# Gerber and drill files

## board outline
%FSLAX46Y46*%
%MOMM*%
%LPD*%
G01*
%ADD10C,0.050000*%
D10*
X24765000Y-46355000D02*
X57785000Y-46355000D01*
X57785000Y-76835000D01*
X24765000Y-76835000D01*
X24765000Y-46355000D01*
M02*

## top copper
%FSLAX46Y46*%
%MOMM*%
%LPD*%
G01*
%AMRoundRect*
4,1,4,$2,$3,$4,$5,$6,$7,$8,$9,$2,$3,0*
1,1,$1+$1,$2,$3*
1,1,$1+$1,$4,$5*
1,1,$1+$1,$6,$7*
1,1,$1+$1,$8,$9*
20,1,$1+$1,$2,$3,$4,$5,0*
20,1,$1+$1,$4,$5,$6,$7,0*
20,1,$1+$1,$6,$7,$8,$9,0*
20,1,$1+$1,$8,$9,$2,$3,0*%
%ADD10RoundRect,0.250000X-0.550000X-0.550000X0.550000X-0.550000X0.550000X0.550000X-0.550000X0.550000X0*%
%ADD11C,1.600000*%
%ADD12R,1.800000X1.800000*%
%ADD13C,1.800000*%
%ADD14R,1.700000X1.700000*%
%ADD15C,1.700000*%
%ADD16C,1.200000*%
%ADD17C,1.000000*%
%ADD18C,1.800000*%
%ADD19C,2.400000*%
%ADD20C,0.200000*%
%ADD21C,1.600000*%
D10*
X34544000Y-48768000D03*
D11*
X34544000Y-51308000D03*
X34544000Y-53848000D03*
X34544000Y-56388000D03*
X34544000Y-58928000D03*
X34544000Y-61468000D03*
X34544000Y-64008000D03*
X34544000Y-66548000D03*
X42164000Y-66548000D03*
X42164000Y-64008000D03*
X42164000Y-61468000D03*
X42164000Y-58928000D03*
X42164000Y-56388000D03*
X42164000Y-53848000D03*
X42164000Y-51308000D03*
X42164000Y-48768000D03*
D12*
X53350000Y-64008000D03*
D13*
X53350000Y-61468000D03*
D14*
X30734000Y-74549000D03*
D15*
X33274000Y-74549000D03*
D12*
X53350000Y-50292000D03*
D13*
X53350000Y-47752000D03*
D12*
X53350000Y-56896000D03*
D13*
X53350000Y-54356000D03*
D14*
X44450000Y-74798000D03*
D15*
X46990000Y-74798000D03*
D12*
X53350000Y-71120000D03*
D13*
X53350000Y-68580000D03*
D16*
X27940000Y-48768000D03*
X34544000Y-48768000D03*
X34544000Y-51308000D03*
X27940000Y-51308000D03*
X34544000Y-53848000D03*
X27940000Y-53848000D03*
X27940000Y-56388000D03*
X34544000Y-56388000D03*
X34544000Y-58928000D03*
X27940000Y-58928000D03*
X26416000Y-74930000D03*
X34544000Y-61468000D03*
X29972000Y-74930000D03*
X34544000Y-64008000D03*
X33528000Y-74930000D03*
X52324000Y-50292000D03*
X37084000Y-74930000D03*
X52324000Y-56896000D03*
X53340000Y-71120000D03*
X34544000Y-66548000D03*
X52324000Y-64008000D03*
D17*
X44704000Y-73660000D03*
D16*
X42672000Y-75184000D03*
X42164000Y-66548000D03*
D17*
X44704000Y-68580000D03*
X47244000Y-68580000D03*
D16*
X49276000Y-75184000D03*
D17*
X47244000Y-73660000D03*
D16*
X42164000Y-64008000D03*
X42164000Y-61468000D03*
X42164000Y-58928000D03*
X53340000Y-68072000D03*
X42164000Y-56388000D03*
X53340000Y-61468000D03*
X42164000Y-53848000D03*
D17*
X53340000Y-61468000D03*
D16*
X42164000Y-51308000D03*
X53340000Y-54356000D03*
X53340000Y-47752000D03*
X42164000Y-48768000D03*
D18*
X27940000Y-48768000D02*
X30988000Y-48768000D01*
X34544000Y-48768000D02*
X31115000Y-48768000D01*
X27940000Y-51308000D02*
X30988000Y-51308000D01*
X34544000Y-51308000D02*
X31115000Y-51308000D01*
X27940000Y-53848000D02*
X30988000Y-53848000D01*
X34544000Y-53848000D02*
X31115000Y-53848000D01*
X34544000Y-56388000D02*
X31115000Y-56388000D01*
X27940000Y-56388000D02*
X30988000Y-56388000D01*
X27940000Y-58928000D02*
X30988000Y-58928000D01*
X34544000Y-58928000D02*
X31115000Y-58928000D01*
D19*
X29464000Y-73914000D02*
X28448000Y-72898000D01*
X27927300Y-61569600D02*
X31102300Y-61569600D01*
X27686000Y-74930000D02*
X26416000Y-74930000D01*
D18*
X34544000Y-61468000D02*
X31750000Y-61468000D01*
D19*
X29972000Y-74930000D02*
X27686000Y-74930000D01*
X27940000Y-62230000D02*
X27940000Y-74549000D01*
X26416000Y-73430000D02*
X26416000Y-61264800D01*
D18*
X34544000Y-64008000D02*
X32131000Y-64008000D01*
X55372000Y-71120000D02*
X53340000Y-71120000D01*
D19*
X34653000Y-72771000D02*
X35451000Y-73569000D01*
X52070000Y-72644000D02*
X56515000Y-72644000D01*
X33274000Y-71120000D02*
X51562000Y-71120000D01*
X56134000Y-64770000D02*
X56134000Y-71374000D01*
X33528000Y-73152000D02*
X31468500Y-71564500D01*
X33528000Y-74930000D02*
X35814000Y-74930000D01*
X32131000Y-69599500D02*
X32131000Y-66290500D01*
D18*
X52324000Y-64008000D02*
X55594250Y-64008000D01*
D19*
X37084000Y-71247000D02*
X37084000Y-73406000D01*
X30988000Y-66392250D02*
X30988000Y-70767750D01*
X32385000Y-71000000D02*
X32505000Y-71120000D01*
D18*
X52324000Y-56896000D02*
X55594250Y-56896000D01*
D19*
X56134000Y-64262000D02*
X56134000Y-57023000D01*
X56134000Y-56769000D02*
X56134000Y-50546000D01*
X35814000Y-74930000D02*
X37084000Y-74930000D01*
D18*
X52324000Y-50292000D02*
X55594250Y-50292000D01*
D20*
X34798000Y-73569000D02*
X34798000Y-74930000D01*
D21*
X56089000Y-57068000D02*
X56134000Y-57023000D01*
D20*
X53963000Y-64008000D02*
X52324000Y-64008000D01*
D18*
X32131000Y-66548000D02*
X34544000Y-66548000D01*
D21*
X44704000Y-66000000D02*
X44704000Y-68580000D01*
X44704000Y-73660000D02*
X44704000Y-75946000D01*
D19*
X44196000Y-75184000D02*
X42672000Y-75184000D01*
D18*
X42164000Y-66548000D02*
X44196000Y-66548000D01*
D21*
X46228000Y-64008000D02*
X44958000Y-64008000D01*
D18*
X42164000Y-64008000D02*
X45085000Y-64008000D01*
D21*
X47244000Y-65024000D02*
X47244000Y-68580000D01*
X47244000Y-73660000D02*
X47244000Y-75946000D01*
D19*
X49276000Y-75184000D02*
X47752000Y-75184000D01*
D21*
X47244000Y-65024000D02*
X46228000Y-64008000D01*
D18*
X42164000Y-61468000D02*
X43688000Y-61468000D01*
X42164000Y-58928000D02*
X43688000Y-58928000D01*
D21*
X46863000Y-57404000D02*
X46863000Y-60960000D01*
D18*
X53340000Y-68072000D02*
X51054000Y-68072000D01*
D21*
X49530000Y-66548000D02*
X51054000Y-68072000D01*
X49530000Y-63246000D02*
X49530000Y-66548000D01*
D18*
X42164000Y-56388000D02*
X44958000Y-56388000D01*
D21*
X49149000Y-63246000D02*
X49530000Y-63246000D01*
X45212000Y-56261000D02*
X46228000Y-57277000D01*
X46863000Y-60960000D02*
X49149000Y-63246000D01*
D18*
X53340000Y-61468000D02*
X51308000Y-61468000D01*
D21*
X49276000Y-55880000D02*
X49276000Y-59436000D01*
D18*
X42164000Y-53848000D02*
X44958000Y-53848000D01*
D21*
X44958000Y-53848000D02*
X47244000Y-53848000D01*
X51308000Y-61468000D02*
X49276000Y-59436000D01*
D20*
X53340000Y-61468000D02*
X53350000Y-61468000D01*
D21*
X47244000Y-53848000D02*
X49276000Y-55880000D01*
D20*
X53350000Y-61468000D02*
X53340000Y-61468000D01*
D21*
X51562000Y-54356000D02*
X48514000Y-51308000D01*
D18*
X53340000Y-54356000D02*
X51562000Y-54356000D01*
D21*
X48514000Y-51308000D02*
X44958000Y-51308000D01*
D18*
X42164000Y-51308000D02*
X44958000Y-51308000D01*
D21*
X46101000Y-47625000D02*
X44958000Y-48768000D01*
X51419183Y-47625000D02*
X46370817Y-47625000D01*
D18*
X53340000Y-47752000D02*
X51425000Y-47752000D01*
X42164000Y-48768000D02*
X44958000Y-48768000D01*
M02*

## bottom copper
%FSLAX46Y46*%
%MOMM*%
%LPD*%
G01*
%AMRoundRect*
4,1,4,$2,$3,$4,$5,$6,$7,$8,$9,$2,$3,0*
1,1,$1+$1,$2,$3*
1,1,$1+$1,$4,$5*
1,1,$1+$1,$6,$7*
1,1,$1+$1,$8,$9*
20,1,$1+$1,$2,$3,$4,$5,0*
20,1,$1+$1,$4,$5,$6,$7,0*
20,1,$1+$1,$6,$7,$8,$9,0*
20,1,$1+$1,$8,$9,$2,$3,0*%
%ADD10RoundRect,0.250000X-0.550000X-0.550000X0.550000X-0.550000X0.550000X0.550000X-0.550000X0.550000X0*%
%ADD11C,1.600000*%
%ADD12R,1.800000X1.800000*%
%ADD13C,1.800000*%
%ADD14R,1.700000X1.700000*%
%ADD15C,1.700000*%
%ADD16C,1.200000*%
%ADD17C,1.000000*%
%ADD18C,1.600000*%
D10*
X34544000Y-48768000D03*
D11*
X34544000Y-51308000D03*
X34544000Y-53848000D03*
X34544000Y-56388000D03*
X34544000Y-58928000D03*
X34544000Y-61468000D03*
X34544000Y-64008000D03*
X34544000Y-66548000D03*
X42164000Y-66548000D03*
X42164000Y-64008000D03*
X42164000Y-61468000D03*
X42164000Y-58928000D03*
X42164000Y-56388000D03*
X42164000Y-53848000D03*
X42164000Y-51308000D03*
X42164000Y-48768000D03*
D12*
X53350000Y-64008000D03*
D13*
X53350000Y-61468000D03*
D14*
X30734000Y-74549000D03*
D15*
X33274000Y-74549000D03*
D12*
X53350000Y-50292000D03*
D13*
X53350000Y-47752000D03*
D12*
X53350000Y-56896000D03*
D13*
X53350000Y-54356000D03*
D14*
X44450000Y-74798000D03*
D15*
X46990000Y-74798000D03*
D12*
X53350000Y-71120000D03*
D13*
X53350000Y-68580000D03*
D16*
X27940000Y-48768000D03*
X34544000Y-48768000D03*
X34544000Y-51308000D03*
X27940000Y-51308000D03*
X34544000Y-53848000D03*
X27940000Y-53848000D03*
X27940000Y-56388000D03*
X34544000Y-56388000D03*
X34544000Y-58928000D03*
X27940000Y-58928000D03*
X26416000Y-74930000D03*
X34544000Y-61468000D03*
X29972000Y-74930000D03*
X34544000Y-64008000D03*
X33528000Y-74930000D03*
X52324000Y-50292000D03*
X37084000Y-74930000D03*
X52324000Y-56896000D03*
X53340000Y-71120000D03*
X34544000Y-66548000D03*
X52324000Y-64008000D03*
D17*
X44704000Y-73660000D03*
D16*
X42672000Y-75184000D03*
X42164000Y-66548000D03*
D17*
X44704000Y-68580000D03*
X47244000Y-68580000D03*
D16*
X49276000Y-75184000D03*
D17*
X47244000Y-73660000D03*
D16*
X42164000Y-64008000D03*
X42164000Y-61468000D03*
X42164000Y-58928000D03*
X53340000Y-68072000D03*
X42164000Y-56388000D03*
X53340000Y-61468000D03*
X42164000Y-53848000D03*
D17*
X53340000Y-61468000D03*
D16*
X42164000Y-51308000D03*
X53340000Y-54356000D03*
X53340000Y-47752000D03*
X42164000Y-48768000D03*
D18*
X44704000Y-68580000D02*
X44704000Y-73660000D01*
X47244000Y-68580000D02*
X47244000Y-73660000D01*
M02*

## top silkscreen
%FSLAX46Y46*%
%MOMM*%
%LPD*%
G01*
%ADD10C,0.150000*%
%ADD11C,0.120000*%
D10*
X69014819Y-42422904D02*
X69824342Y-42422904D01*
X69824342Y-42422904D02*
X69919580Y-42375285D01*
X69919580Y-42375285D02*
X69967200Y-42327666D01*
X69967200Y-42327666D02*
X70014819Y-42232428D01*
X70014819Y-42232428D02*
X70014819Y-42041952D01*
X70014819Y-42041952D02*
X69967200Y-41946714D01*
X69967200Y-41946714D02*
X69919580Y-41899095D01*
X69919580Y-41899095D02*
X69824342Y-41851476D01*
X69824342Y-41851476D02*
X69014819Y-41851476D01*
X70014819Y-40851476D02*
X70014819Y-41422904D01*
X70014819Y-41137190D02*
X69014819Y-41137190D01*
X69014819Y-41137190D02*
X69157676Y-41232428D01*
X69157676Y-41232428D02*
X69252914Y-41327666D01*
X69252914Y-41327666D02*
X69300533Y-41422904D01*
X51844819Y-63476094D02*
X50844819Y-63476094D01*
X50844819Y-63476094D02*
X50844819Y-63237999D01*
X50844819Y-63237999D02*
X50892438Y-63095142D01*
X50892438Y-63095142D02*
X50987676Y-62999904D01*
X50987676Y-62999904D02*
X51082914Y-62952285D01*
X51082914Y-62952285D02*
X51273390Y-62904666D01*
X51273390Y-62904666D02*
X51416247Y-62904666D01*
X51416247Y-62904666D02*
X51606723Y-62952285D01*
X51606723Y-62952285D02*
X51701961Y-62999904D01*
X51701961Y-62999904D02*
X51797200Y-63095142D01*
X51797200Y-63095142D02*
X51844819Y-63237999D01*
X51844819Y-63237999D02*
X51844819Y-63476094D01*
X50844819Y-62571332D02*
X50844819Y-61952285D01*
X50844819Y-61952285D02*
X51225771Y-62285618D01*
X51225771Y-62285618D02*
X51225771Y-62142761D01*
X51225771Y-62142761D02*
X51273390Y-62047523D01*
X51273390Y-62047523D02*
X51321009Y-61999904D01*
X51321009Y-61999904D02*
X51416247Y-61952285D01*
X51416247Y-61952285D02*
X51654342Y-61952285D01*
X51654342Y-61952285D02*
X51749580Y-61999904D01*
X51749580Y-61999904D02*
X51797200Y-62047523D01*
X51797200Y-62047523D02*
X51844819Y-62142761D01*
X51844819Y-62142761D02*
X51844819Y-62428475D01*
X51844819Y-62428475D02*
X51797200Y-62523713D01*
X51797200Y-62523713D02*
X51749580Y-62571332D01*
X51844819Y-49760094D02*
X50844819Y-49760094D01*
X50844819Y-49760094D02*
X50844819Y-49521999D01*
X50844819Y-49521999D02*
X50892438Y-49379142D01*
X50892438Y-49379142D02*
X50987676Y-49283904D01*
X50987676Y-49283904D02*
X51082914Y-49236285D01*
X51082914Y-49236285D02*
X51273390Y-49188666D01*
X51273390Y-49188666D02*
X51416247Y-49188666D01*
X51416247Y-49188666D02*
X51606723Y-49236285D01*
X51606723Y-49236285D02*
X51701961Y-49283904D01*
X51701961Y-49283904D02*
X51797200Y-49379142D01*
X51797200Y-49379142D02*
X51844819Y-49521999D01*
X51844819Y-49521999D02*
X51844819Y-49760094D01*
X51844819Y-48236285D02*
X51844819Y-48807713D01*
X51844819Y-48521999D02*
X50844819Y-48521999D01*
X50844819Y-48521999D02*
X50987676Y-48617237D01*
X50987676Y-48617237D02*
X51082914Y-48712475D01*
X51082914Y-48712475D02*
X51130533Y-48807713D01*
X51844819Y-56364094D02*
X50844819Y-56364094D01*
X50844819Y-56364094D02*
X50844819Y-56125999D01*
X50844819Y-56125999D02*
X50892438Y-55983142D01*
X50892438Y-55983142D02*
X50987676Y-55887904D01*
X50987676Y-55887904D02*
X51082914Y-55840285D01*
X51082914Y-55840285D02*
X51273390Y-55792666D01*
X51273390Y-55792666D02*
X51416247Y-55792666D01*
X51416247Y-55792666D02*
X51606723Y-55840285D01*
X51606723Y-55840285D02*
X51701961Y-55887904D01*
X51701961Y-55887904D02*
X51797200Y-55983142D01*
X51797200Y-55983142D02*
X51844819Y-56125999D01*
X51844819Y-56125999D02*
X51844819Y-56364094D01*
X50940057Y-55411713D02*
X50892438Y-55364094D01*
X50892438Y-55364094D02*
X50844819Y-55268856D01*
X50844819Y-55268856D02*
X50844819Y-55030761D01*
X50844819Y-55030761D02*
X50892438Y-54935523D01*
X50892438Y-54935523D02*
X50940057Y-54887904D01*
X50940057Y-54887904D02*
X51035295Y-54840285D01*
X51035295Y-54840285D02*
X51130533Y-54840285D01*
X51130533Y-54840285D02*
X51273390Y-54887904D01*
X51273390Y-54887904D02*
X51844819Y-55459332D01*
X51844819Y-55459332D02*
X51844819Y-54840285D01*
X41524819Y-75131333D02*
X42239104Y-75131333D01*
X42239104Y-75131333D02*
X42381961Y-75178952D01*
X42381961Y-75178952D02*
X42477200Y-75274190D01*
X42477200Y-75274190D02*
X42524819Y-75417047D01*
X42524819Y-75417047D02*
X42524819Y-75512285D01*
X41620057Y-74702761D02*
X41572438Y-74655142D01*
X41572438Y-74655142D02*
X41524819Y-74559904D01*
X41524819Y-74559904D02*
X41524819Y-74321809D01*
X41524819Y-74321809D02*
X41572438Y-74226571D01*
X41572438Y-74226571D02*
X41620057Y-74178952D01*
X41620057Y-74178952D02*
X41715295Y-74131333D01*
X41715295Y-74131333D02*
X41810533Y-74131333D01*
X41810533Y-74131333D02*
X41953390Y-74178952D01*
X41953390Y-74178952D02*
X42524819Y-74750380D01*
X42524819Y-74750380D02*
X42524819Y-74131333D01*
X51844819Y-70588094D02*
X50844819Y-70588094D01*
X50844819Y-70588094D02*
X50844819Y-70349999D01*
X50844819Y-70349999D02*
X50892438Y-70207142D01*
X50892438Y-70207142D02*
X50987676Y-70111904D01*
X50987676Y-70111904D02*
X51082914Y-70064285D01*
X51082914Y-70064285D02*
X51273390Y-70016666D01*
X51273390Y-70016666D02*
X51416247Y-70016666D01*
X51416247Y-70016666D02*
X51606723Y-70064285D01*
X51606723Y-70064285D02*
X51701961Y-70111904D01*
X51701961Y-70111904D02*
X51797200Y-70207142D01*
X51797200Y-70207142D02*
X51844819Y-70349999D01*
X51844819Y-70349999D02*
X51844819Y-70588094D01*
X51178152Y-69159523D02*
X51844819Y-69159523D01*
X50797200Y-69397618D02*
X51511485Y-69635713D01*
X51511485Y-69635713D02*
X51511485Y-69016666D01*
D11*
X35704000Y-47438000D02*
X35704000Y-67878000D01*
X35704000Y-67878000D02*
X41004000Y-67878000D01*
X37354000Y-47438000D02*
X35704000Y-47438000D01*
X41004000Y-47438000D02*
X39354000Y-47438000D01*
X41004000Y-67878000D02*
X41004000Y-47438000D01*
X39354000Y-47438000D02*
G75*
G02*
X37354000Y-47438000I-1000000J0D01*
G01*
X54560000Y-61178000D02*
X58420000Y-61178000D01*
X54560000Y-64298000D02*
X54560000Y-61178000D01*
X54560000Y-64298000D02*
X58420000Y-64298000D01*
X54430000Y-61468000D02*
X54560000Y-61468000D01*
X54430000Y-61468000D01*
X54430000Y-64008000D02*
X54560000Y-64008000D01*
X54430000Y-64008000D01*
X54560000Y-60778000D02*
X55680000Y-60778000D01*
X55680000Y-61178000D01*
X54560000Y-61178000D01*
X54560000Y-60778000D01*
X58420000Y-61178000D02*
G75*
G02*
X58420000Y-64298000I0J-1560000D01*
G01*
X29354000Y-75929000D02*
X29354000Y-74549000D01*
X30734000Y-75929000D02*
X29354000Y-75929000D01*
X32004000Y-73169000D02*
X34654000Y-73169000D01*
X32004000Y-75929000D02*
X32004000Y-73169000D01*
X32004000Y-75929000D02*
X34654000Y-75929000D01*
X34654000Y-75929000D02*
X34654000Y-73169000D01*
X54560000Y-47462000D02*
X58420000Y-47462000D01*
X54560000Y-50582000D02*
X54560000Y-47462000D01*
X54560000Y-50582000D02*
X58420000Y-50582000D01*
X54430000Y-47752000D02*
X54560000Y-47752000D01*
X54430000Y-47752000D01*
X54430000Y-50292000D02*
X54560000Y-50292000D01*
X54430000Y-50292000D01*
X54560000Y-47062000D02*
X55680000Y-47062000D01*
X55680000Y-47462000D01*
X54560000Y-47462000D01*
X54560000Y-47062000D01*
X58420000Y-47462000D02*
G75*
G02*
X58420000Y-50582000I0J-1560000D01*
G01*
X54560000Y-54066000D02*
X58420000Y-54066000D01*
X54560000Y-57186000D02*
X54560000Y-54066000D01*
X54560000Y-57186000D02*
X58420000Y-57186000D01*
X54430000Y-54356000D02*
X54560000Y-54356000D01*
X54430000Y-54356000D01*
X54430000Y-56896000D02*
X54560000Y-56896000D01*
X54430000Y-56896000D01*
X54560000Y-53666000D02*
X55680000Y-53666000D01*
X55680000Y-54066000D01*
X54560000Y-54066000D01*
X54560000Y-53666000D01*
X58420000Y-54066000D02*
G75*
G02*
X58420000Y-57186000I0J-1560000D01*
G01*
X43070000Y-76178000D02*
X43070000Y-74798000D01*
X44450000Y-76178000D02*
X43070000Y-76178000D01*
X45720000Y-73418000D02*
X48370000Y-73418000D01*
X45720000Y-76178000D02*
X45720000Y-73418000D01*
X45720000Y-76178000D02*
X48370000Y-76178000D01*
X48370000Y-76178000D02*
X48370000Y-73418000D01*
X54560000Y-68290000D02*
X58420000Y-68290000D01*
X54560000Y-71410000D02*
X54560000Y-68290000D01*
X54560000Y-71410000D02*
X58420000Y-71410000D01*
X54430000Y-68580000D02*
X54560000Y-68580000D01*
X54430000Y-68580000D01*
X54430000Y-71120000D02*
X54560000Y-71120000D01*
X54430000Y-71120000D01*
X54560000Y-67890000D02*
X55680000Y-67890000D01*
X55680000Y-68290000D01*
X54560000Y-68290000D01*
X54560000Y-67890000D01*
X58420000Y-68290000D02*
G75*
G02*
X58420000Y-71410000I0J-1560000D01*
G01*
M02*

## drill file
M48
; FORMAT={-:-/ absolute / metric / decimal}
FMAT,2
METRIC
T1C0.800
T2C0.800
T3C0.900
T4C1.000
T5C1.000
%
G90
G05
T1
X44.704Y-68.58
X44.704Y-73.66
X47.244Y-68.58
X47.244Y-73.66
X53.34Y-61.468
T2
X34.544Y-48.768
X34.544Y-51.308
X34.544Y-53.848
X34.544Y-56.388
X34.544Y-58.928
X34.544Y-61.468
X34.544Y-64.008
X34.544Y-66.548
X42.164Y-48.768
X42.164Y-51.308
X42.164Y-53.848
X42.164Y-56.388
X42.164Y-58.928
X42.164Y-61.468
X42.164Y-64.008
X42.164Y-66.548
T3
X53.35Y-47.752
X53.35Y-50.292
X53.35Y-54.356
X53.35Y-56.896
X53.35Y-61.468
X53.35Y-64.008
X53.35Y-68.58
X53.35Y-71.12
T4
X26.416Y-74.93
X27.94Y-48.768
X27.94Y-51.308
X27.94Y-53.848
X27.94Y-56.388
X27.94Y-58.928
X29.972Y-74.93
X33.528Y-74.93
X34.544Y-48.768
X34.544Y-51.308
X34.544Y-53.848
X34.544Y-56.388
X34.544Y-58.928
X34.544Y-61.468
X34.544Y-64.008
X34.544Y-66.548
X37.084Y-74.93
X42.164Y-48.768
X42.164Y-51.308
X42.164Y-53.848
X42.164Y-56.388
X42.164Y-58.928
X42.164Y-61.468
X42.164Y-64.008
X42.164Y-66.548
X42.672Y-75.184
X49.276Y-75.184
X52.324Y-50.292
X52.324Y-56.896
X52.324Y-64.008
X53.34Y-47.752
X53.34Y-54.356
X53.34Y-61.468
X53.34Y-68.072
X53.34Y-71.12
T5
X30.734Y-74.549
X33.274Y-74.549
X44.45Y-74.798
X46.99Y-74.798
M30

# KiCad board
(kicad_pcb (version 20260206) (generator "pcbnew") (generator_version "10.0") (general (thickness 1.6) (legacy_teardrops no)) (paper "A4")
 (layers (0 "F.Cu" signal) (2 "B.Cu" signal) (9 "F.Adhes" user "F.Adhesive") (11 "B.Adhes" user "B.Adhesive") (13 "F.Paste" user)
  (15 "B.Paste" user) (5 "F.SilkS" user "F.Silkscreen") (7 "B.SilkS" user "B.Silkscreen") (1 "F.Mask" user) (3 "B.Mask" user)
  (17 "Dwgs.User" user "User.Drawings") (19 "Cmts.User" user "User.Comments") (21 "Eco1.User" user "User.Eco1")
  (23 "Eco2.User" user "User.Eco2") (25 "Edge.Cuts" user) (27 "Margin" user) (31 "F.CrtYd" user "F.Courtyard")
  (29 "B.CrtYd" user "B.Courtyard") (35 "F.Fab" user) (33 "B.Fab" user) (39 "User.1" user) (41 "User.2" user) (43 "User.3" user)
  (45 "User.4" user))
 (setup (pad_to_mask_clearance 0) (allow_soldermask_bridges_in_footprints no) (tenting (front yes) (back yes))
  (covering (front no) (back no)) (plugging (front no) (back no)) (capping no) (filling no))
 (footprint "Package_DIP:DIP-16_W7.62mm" (layer "F.Cu") (at 34.544 48.768)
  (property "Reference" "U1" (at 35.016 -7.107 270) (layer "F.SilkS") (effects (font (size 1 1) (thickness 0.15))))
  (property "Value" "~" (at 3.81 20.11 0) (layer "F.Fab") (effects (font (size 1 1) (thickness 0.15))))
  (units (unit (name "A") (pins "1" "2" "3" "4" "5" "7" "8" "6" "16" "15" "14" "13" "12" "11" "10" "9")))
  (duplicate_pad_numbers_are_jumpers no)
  (fp_line (start 1.16 -1.33) (end 1.16 19.11) (stroke (width 0.12) (type solid)) (layer "F.SilkS"))
  (fp_line (start 1.16 19.11) (end 6.46 19.11) (stroke (width 0.12) (type solid)) (layer "F.SilkS"))
  (fp_line (start 2.81 -1.33) (end 1.16 -1.33) (stroke (width 0.12) (type solid)) (layer "F.SilkS"))
  (fp_line (start 6.46 -1.33) (end 4.81 -1.33) (stroke (width 0.12) (type solid)) (layer "F.SilkS"))
  (fp_line (start 6.46 19.11) (end 6.46 -1.33) (stroke (width 0.12) (type solid)) (layer "F.SilkS"))
  (fp_arc (start 4.81 -1.33) (mid 3.81 -0.33) (end 2.81 -1.33) (stroke (width 0.12) (type solid)) (layer "F.SilkS"))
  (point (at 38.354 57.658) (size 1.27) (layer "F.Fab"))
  (pad "1" thru_hole roundrect (at 0 0) (size 1.6 1.6) (drill 0.8) (layers "*.Cu" "*.Mask") (remove_unused_layers no)
   (roundrect_rratio 0.15625) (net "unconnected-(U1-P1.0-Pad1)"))
  (pad "2" thru_hole circle (at 0 2.54) (size 1.6 1.6) (drill 0.8) (layers "*.Cu" "*.Mask") (remove_unused_layers no)
   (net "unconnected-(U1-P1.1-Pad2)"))
  (pad "3" thru_hole circle (at 0 5.08) (size 1.6 1.6) (drill 0.8) (layers "*.Cu" "*.Mask") (remove_unused_layers no)
   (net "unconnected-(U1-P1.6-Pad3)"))
  (pad "4" thru_hole circle (at 0 7.62) (size 1.6 1.6) (drill 0.8) (layers "*.Cu" "*.Mask") (remove_unused_layers no)
   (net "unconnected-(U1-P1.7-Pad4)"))
  (pad "5" thru_hole circle (at 0 10.16) (size 1.6 1.6) (drill 0.8) (layers "*.Cu" "*.Mask") (remove_unused_layers no)
   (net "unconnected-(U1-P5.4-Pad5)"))
  (pad "6" thru_hole circle (at 0 12.7) (size 1.6 1.6) (drill 0.8) (layers "*.Cu" "*.Mask") (remove_unused_layers no) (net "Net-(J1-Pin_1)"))
  (pad "7" thru_hole circle (at 0 15.24) (size 1.6 1.6) (drill 0.8) (layers "*.Cu" "*.Mask") (remove_unused_layers no)
   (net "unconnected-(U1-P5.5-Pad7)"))
  (pad "8" thru_hole circle (at 0 17.78) (size 1.6 1.6) (drill 0.8) (layers "*.Cu" "*.Mask") (remove_unused_layers no) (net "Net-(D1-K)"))
  (pad "9" thru_hole circle (at 7.62 17.78) (size 1.6 1.6) (drill 0.8) (layers "*.Cu" "*.Mask") (remove_unused_layers no)
   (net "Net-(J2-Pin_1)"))
  (pad "10" thru_hole circle (at 7.62 15.24) (size 1.6 1.6) (drill 0.8) (layers "*.Cu" "*.Mask") (remove_unused_layers no)
   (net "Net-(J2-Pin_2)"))
  (pad "11" thru_hole circle (at 7.62 12.7) (size 1.6 1.6) (drill 0.8) (layers "*.Cu" "*.Mask") (remove_unused_layers no)
   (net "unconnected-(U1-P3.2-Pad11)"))
  (pad "12" thru_hole circle (at 7.62 10.16) (size 1.6 1.6) (drill 0.8) (layers "*.Cu" "*.Mask") (remove_unused_layers no)
   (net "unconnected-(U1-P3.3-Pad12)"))
  (pad "13" thru_hole circle (at 7.62 7.62) (size 1.6 1.6) (drill 0.8) (layers "*.Cu" "*.Mask") (remove_unused_layers no) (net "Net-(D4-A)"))
  (pad "14" thru_hole circle (at 7.62 5.08) (size 1.6 1.6) (drill 0.8) (layers "*.Cu" "*.Mask") (remove_unused_layers no) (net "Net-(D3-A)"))
  (pad "15" thru_hole circle (at 7.62 2.54) (size 1.6 1.6) (drill 0.8) (layers "*.Cu" "*.Mask") (remove_unused_layers no) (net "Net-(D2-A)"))
  (pad "16" thru_hole circle (at 7.62 0) (size 1.6 1.6) (drill 0.8) (layers "*.Cu" "*.Mask") (remove_unused_layers no) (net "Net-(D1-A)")))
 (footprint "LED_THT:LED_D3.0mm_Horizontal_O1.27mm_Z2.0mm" (layer "F.Cu") (at 53.35 64.008 90)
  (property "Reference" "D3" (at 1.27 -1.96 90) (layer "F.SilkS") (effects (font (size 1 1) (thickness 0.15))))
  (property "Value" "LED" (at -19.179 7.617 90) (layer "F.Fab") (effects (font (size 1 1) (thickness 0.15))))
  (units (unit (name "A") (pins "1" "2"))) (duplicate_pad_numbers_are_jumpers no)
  (fp_line (start 2.83 1.21) (end 2.83 5.07) (stroke (width 0.12) (type solid)) (layer "F.SilkS"))
  (fp_line (start -0.29 1.21) (end 2.83 1.21) (stroke (width 0.12) (type solid)) (layer "F.SilkS"))
  (fp_line (start -0.29 1.21) (end -0.29 5.07) (stroke (width 0.12) (type solid)) (layer "F.SilkS"))
  (fp_rect (start 2.54 1.08) (end 2.54 1.21) (stroke (width 0.12) (type solid)) (fill no) (layer "F.SilkS"))
  (fp_rect (start 0 1.08) (end 0 1.21) (stroke (width 0.12) (type solid)) (fill no) (layer "F.SilkS"))
  (fp_rect (start 2.83 1.21) (end 3.23 2.33) (stroke (width 0.12) (type solid)) (fill no) (layer "F.SilkS"))
  (fp_arc (start 2.83 5.07) (mid 1.27 6.63) (end -0.29 5.07) (stroke (width 0.12) (type solid)) (layer "F.SilkS"))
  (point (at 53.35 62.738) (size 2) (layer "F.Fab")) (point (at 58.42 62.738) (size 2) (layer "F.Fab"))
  (pad "1" thru_hole rect (at 0 0 90) (size 1.8 1.8) (drill 0.9) (layers "*.Cu" "*.Mask") (remove_unused_layers no) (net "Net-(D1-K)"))
  (pad "2" thru_hole circle (at 2.54 0 90) (size 1.8 1.8) (drill 0.9) (layers "*.Cu" "*.Mask") (remove_unused_layers no) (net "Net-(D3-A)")))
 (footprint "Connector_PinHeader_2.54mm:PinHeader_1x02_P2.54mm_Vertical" (layer "F.Cu") (at 30.734 74.549 90)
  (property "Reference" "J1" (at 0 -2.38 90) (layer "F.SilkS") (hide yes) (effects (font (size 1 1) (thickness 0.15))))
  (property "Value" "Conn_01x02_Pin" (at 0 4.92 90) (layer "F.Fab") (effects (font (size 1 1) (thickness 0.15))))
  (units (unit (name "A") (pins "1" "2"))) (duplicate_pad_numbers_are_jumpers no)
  (fp_line (start -1.38 -1.38) (end 0 -1.38) (stroke (width 0.12) (type solid)) (layer "F.SilkS"))
  (fp_line (start -1.38 0) (end -1.38 -1.38) (stroke (width 0.12) (type solid)) (layer "F.SilkS"))
  (fp_line (start 1.38 1.27) (end 1.38 3.92) (stroke (width 0.12) (type solid)) (layer "F.SilkS"))
  (fp_line (start -1.38 1.27) (end 1.38 1.27) (stroke (width 0.12) (type solid)) (layer "F.SilkS"))
  (fp_line (start -1.38 1.27) (end -1.38 3.92) (stroke (width 0.12) (type solid)) (layer "F.SilkS"))
  (fp_line (start -1.38 3.92) (end 1.38 3.92) (stroke (width 0.12) (type solid)) (layer "F.SilkS"))
  (pad "1" thru_hole rect (at 0 0 90) (size 1.7 1.7) (drill 1) (layers "*.Cu" "*.Mask") (remove_unused_layers no) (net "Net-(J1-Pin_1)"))
  (pad "2" thru_hole circle (at 0 2.54 90) (size 1.7 1.7) (drill 1) (layers "*.Cu" "*.Mask") (remove_unused_layers no) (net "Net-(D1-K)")))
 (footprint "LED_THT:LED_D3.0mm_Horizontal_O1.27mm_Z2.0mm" (layer "F.Cu") (at 53.35 50.292 90)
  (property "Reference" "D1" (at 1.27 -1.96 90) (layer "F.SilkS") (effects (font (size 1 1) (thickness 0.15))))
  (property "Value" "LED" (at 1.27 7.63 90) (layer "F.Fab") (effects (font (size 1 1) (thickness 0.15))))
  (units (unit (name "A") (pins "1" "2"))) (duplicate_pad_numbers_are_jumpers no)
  (fp_line (start 2.83 1.21) (end 2.83 5.07) (stroke (width 0.12) (type solid)) (layer "F.SilkS"))
  (fp_line (start -0.29 1.21) (end 2.83 1.21) (stroke (width 0.12) (type solid)) (layer "F.SilkS"))
  (fp_line (start -0.29 1.21) (end -0.29 5.07) (stroke (width 0.12) (type solid)) (layer "F.SilkS"))
  (fp_rect (start 2.54 1.08) (end 2.54 1.21) (stroke (width 0.12) (type solid)) (fill no) (layer "F.SilkS"))
  (fp_rect (start 0 1.08) (end 0 1.21) (stroke (width 0.12) (type solid)) (fill no) (layer "F.SilkS"))
  (fp_rect (start 2.83 1.21) (end 3.23 2.33) (stroke (width 0.12) (type solid)) (fill no) (layer "F.SilkS"))
  (fp_arc (start 2.83 5.07) (mid 1.27 6.63) (end -0.29 5.07) (stroke (width 0.12) (type solid)) (layer "F.SilkS"))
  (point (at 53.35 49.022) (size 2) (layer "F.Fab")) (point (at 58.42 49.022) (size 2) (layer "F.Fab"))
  (pad "1" thru_hole rect (at 0 0 90) (size 1.8 1.8) (drill 0.9) (layers "*.Cu" "*.Mask") (remove_unused_layers no) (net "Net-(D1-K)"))
  (pad "2" thru_hole circle (at 2.54 0 90) (size 1.8 1.8) (drill 0.9) (layers "*.Cu" "*.Mask") (remove_unused_layers no) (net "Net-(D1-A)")))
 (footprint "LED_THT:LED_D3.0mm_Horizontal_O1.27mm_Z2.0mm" (layer "F.Cu") (at 53.35 56.896 90)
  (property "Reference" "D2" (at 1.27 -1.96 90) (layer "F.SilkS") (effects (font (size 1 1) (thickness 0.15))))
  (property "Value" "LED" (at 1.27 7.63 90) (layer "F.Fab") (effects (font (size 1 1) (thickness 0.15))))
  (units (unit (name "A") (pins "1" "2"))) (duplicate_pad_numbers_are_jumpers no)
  (fp_line (start 2.83 1.21) (end 2.83 5.07) (stroke (width 0.12) (type solid)) (layer "F.SilkS"))
  (fp_line (start -0.29 1.21) (end 2.83 1.21) (stroke (width 0.12) (type solid)) (layer "F.SilkS"))
  (fp_line (start -0.29 1.21) (end -0.29 5.07) (stroke (width 0.12) (type solid)) (layer "F.SilkS"))
  (fp_rect (start 2.54 1.08) (end 2.54 1.21) (stroke (width 0.12) (type solid)) (fill no) (layer "F.SilkS"))
  (fp_rect (start 0 1.08) (end 0 1.21) (stroke (width 0.12) (type solid)) (fill no) (layer "F.SilkS"))
  (fp_rect (start 2.83 1.21) (end 3.23 2.33) (stroke (width 0.12) (type solid)) (fill no) (layer "F.SilkS"))
  (fp_arc (start 2.83 5.07) (mid 1.27 6.63) (end -0.29 5.07) (stroke (width 0.12) (type solid)) (layer "F.SilkS"))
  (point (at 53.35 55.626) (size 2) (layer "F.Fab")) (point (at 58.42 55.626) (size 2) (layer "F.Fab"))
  (pad "1" thru_hole rect (at 0 0 90) (size 1.8 1.8) (drill 0.9) (layers "*.Cu" "*.Mask") (remove_unused_layers no) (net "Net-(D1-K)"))
  (pad "2" thru_hole circle (at 2.54 0 90) (size 1.8 1.8) (drill 0.9) (layers "*.Cu" "*.Mask") (remove_unused_layers no) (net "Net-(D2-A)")))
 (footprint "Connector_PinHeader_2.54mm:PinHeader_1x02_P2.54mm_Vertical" (layer "F.Cu") (at 44.45 74.798 90)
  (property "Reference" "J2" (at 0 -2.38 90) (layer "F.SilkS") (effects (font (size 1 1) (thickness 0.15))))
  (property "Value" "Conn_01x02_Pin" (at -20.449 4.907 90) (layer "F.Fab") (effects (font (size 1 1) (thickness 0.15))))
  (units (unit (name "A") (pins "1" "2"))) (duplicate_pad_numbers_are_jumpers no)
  (fp_line (start -1.38 -1.38) (end 0 -1.38) (stroke (width 0.12) (type solid)) (layer "F.SilkS"))
  (fp_line (start -1.38 0) (end -1.38 -1.38) (stroke (width 0.12) (type solid)) (layer "F.SilkS"))
  (fp_line (start 1.38 1.27) (end 1.38 3.92) (stroke (width 0.12) (type solid)) (layer "F.SilkS"))
  (fp_line (start -1.38 1.27) (end 1.38 1.27) (stroke (width 0.12) (type solid)) (layer "F.SilkS"))
  (fp_line (start -1.38 1.27) (end -1.38 3.92) (stroke (width 0.12) (type solid)) (layer "F.SilkS"))
  (fp_line (start -1.38 3.92) (end 1.38 3.92) (stroke (width 0.12) (type solid)) (layer "F.SilkS"))
  (pad "1" thru_hole rect (at 0 0 90) (size 1.7 1.7) (drill 1) (layers "*.Cu" "*.Mask") (remove_unused_layers no) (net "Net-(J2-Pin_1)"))
  (pad "2" thru_hole circle (at 0 2.54 90) (size 1.7 1.7) (drill 1) (layers "*.Cu" "*.Mask") (remove_unused_layers no)
   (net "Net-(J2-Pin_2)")))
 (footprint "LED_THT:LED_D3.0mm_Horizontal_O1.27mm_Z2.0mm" (layer "F.Cu") (at 53.35 71.12 90)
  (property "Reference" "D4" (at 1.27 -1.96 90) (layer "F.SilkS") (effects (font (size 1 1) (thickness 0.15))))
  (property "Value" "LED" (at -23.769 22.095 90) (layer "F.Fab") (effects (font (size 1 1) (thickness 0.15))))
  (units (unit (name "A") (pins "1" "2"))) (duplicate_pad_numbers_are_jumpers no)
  (fp_line (start 2.83 1.21) (end 2.83 5.07) (stroke (width 0.12) (type solid)) (layer "F.SilkS"))
  (fp_line (start -0.29 1.21) (end 2.83 1.21) (stroke (width 0.12) (type solid)) (layer "F.SilkS"))
  (fp_line (start -0.29 1.21) (end -0.29 5.07) (stroke (width 0.12) (type solid)) (layer "F.SilkS"))
  (fp_rect (start 2.54 1.08) (end 2.54 1.21) (stroke (width 0.12) (type solid)) (fill no) (layer "F.SilkS"))
  (fp_rect (start 0 1.08) (end 0 1.21) (stroke (width 0.12) (type solid)) (fill no) (layer "F.SilkS"))
  (fp_rect (start 2.83 1.21) (end 3.23 2.33) (stroke (width 0.12) (type solid)) (fill no) (layer "F.SilkS"))
  (fp_arc (start 2.83 5.07) (mid 1.27 6.63) (end -0.29 5.07) (stroke (width 0.12) (type solid)) (layer "F.SilkS"))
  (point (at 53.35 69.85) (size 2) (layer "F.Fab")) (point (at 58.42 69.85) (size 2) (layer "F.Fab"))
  (pad "1" thru_hole rect (at 0 0 90) (size 1.8 1.8) (drill 0.9) (layers "*.Cu" "*.Mask") (remove_unused_layers no) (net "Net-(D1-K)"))
  (pad "2" thru_hole circle (at 2.54 0 90) (size 1.8 1.8) (drill 0.9) (layers "*.Cu" "*.Mask") (remove_unused_layers no) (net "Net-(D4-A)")))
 (gr_rect (start 24.765 46.355) (end 57.785 76.835) (stroke (width 0.05) (type default)) (fill no) (layer "Edge.Cuts"))
 (segment (start 27.94 48.768) (end 30.988 48.768) (width 1.8) (layer "F.Cu") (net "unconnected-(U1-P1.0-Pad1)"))
 (segment (start 34.544 48.768) (end 31.115 48.768) (width 1.8) (layer "F.Cu") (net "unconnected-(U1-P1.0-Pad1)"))
 (via (at 27.94 48.768) (size 1.2) (drill 1) (layers "F.Cu" "B.Cu") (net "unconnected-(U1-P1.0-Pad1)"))
 (via (at 34.544 48.768) (size 1.2) (drill 1) (layers "F.Cu" "B.Cu") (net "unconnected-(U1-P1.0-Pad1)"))
 (segment (start 27.94 51.308) (end 30.988 51.308) (width 1.8) (layer "F.Cu") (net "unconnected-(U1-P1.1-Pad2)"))
 (segment (start 34.544 51.308) (end 31.115 51.308) (width 1.8) (layer "F.Cu") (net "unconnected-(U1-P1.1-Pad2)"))
 (via (at 34.544 51.308) (size 1.2) (drill 1) (layers "F.Cu" "B.Cu") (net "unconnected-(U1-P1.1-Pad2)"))
 (via (at 27.94 51.308) (size 1.2) (drill 1) (layers "F.Cu" "B.Cu") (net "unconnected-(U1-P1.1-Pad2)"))
 (segment (start 27.94 53.848) (end 30.988 53.848) (width 1.8) (layer "F.Cu") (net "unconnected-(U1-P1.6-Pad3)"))
 (segment (start 34.544 53.848) (end 31.115 53.848) (width 1.8) (layer "F.Cu") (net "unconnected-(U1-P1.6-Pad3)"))
 (via (at 34.544 53.848) (size 1.2) (drill 1) (layers "F.Cu" "B.Cu") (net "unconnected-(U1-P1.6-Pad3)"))
 (via (at 27.94 53.848) (size 1.2) (drill 1) (layers "F.Cu" "B.Cu") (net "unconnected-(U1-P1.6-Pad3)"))
 (segment (start 34.544 56.388) (end 31.115 56.388) (width 1.8) (layer "F.Cu") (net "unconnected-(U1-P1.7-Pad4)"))
 (segment (start 27.94 56.388) (end 30.988 56.388) (width 1.8) (layer "F.Cu") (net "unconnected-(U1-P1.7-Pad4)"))
 (via (at 27.94 56.388) (size 1.2) (drill 1) (layers "F.Cu" "B.Cu") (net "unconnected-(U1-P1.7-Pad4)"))
 (via (at 34.544 56.388) (size 1.2) (drill 1) (layers "F.Cu" "B.Cu") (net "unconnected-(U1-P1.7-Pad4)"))
 (segment (start 27.94 58.928) (end 30.988 58.928) (width 1.8) (layer "F.Cu") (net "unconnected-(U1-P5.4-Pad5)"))
 (segment (start 34.544 58.928) (end 31.115 58.928) (width 1.8) (layer "F.Cu") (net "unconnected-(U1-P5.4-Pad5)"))
 (via (at 34.544 58.928) (size 1.2) (drill 1) (layers "F.Cu" "B.Cu") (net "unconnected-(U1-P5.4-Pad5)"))
 (via (at 27.94 58.928) (size 1.2) (drill 1) (layers "F.Cu" "B.Cu") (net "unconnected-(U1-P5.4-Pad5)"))
 (segment (start 29.464 73.914) (end 28.448 72.898) (width 2.4) (layer "F.Cu") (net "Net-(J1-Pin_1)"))
 (segment (start 27.9273 61.5696) (end 31.1023 61.5696) (width 2.4) (layer "F.Cu") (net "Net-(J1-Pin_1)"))
 (segment (start 27.686 74.93) (end 26.416 74.93) (width 2.4) (layer "F.Cu") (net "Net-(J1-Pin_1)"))
 (segment (start 34.544 61.468) (end 31.75 61.468) (width 1.8) (layer "F.Cu") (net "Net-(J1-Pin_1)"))
 (segment (start 29.972 74.93) (end 27.686 74.93) (width 2.4) (layer "F.Cu") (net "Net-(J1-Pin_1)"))
 (segment (start 27.94 62.23) (end 27.94 74.549) (width 2.4) (layer "F.Cu") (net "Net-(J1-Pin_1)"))
 (segment (start 26.416 73.43) (end 26.416 61.2648) (width 2.4) (layer "F.Cu") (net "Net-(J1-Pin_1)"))
 (via (at 26.416 74.93) (size 1.2) (drill 1) (layers "F.Cu" "B.Cu") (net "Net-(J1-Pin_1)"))
 (via (at 34.544 61.468) (size 1.2) (drill 1) (layers "F.Cu" "B.Cu") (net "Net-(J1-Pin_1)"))
 (via (at 29.972 74.93) (size 1.2) (drill 1) (layers "F.Cu" "B.Cu") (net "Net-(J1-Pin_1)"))
 (segment (start 34.544 64.008) (end 32.131 64.008) (width 1.8) (layer "F.Cu") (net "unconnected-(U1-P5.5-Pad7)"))
 (via (at 34.544 64.008) (size 1.2) (drill 1) (layers "F.Cu" "B.Cu") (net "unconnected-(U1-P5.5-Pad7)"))
 (segment (start 55.372 71.12) (end 53.34 71.12) (width 1.8) (layer "F.Cu") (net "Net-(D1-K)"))
 (segment (start 34.653 72.771) (end 35.451 73.569) (width 2.4) (layer "F.Cu") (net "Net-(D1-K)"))
 (segment (start 52.07 72.644) (end 56.515 72.644) (width 2.4) (layer "F.Cu") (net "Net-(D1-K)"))
 (segment (start 33.274 71.12) (end 51.562 71.12) (width 2.4) (layer "F.Cu") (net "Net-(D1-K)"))
 (segment (start 56.134 64.77) (end 56.134 71.374) (width 2.4) (layer "F.Cu") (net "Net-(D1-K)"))
 (segment (start 33.528 73.152) (end 31.4685 71.5645) (width 2.4) (layer "F.Cu") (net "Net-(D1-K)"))
 (segment (start 33.528 74.93) (end 35.814 74.93) (width 2.4) (layer "F.Cu") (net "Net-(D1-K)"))
 (segment (start 32.131 69.5995) (end 32.131 66.2905) (width 2.4) (layer "F.Cu") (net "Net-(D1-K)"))
 (segment (start 52.324 64.008) (end 55.59425 64.008) (width 1.8) (layer "F.Cu") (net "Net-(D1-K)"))
 (segment (start 37.084 71.247) (end 37.084 73.406) (width 2.4) (layer "F.Cu") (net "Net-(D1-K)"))
 (segment (start 30.988 66.39225) (end 30.988 70.76775) (width 2.4) (layer "F.Cu") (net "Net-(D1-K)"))
 (segment (start 32.385 71) (end 32.505 71.12) (width 2.4) (layer "F.Cu") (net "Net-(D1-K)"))
 (segment (start 52.324 56.896) (end 55.59425 56.896) (width 1.8) (layer "F.Cu") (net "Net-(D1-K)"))
 (segment (start 56.134 64.262) (end 56.134 57.023) (width 2.4) (layer "F.Cu") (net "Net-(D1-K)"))
 (segment (start 56.134 56.769) (end 56.134 50.546) (width 2.4) (layer "F.Cu") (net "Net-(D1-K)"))
 (segment (start 35.814 74.93) (end 37.084 74.93) (width 2.4) (layer "F.Cu") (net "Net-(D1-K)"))
 (segment (start 52.324 50.292) (end 55.59425 50.292) (width 1.8) (layer "F.Cu") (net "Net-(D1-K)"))
 (segment (start 34.798 73.569) (end 34.798 74.93) (width 0.2) (layer "F.Cu") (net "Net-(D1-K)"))
 (segment (start 56.089 57.068) (end 56.134 57.023) (width 1.6) (layer "F.Cu") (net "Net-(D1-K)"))
 (segment (start 53.963 64.008) (end 52.324 64.008) (width 0.2) (layer "F.Cu") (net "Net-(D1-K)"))
 (segment (start 32.131 66.548) (end 34.544 66.548) (width 1.8) (layer "F.Cu") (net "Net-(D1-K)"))
 (via (at 33.528 74.93) (size 1.2) (drill 1) (layers "F.Cu" "B.Cu") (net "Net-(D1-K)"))
 (via (at 52.324 50.292) (size 1.2) (drill 1) (layers "F.Cu" "B.Cu") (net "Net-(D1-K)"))
 (via (at 37.084 74.93) (size 1.2) (drill 1) (layers "F.Cu" "B.Cu") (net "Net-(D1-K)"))
 (via (at 52.324 56.896) (size 1.2) (drill 1) (layers "F.Cu" "B.Cu") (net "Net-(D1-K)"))
 (via (at 53.34 71.12) (size 1.2) (drill 1) (layers "F.Cu" "B.Cu") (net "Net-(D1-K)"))
 (via (at 34.544 66.548) (size 1.2) (drill 1) (layers "F.Cu" "B.Cu") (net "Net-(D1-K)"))
 (via (at 52.324 64.008) (size 1.2) (drill 1) (layers "F.Cu" "B.Cu") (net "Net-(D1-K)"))
 (segment (start 44.704 66) (end 44.704 68.58) (width 1.6) (layer "F.Cu") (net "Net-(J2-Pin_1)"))
 (segment (start 44.704 73.66) (end 44.704 75.946) (width 1.6) (layer "F.Cu") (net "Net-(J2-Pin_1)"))
 (segment (start 44.196 75.184) (end 42.672 75.184) (width 2.4) (layer "F.Cu") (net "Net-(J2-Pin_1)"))
 (segment (start 42.164 66.548) (end 44.196 66.548) (width 1.8) (layer "F.Cu") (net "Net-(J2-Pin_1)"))
 (via (at 44.704 73.66) (size 1) (drill 0.8) (layers "F.Cu" "B.Cu") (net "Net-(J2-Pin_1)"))
 (via (at 42.672 75.184) (size 1.2) (drill 1) (layers "F.Cu" "B.Cu") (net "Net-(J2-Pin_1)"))
 (via (at 42.164 66.548) (size 1.2) (drill 1) (layers "F.Cu" "B.Cu") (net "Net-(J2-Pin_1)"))
 (via (at 44.704 68.58) (size 1) (drill 0.8) (layers "F.Cu" "B.Cu") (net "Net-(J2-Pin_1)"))
 (segment (start 44.704 68.58) (end 44.704 73.66) (width 1.6) (layer "B.Cu") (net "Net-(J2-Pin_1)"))
 (segment (start 46.228 64.008) (end 44.958 64.008) (width 1.6) (layer "F.Cu") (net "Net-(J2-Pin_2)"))
 (segment (start 42.164 64.008) (end 45.085 64.008) (width 1.8) (layer "F.Cu") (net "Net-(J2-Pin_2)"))
 (segment (start 47.244 65.024) (end 47.244 68.58) (width 1.6) (layer "F.Cu") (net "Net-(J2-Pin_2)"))
 (segment (start 47.244 73.66) (end 47.244 75.946) (width 1.6) (layer "F.Cu") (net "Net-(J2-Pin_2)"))
 (segment (start 49.276 75.184) (end 47.752 75.184) (width 2.4) (layer "F.Cu") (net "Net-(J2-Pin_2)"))
 (segment (start 47.244 65.024) (end 46.228 64.008) (width 1.6) (layer "F.Cu") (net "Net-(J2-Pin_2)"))
 (via (at 47.244 68.58) (size 1) (drill 0.8) (layers "F.Cu" "B.Cu") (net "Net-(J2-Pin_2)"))
 (via (at 49.276 75.184) (size 1.2) (drill 1) (layers "F.Cu" "B.Cu") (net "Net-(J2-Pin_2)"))
 (via (at 47.244 73.66) (size 1) (drill 0.8) (layers "F.Cu" "B.Cu") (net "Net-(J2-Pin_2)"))
 (via (at 42.164 64.008) (size 1.2) (drill 1) (layers "F.Cu" "B.Cu") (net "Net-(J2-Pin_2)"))
 (segment (start 47.244 68.58) (end 47.244 73.66) (width 1.6) (layer "B.Cu") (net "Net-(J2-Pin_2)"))
 (segment (start 42.164 61.468) (end 43.688 61.468) (width 1.8) (layer "F.Cu") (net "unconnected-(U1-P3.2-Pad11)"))
 (via (at 42.164 61.468) (size 1.2) (drill 1) (layers "F.Cu" "B.Cu") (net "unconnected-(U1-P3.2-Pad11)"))
 (segment (start 42.164 58.928) (end 43.688 58.928) (width 1.8) (layer "F.Cu") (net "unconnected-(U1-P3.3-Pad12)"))
 (via (at 42.164 58.928) (size 1.2) (drill 1) (layers "F.Cu" "B.Cu") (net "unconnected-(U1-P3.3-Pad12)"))
 (segment (start 46.863 57.404) (end 46.863 60.96) (width 1.6) (layer "F.Cu") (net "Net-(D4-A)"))
 (segment (start 53.34 68.072) (end 51.054 68.072) (width 1.8) (layer "F.Cu") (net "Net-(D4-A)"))
 (segment (start 49.53 66.548) (end 51.054 68.072) (width 1.6) (layer "F.Cu") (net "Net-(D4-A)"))
 (segment (start 49.53 63.246) (end 49.53 66.548) (width 1.6) (layer "F.Cu") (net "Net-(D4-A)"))
 (segment (start 42.164 56.388) (end 44.958 56.388) (width 1.8) (layer "F.Cu") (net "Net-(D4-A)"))
 (segment (start 49.149 63.246) (end 49.53 63.246) (width 1.6) (layer "F.Cu") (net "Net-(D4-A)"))
 (segment (start 45.212 56.261) (end 46.228 57.277) (width 1.6) (layer "F.Cu") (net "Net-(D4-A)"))
 (segment (start 46.863 60.96) (end 49.149 63.246) (width 1.6) (layer "F.Cu") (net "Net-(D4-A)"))
 (via (at 53.34 68.072) (size 1.2) (drill 1) (layers "F.Cu" "B.Cu") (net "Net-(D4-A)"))
 (via (at 42.164 56.388) (size 1.2) (drill 1) (layers "F.Cu" "B.Cu") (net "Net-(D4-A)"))
 (segment (start 53.34 61.468) (end 51.308 61.468) (width 1.8) (layer "F.Cu") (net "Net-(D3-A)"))
 (segment (start 49.276 55.88) (end 49.276 59.436) (width 1.6) (layer "F.Cu") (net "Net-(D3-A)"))
 (segment (start 42.164 53.848) (end 44.958 53.848) (width 1.8) (layer "F.Cu") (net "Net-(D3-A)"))
 (segment (start 44.958 53.848) (end 47.244 53.848) (width 1.6) (layer "F.Cu") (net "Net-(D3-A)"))
 (segment (start 51.308 61.468) (end 49.276 59.436) (width 1.6) (layer "F.Cu") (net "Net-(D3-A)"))
 (segment (start 53.34 61.468) (end 53.35 61.468) (width 0.2) (layer "F.Cu") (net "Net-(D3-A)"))
 (segment (start 47.244 53.848) (end 49.276 55.88) (width 1.6) (layer "F.Cu") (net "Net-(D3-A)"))
 (segment (start 53.35 61.468) (end 53.34 61.468) (width 0.2) (layer "F.Cu") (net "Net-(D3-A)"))
 (via (at 53.34 61.468) (size 1.2) (drill 1) (layers "F.Cu" "B.Cu") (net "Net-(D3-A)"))
 (via (at 42.164 53.848) (size 1.2) (drill 1) (layers "F.Cu" "B.Cu") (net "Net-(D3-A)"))
 (via (at 53.34 61.468) (size 1) (drill 0.8) (layers "F.Cu" "B.Cu") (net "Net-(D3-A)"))
 (segment (start 51.562 54.356) (end 48.514 51.308) (width 1.6) (layer "F.Cu") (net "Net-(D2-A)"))
 (segment (start 53.34 54.356) (end 51.562 54.356) (width 1.8) (layer "F.Cu") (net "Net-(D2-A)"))
 (segment (start 48.514 51.308) (end 44.958 51.308) (width 1.6) (layer "F.Cu") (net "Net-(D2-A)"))
 (segment (start 42.164 51.308) (end 44.958 51.308) (width 1.8) (layer "F.Cu") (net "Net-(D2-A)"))
 (via (at 42.164 51.308) (size 1.2) (drill 1) (layers "F.Cu" "B.Cu") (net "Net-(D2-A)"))
 (via (at 53.34 54.356) (size 1.2) (drill 1) (layers "F.Cu" "B.Cu") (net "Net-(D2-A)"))
 (segment (start 46.101 47.625) (end 44.958 48.768) (width 1.6) (layer "F.Cu") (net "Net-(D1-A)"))
 (segment (start 51.419183 47.625) (end 46.370817 47.625) (width 1.6) (layer "F.Cu") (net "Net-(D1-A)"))
 (segment (start 53.34 47.752) (end 51.425 47.752) (width 1.8) (layer "F.Cu") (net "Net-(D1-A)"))
 (segment (start 42.164 48.768) (end 44.958 48.768) (width 1.8) (layer "F.Cu") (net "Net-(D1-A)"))
 (via (at 53.34 47.752) (size 1.2) (drill 1) (layers "F.Cu" "B.Cu") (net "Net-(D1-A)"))
 (via (at 42.164 48.768) (size 1.2) (drill 1) (layers "F.Cu" "B.Cu") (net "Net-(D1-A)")))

